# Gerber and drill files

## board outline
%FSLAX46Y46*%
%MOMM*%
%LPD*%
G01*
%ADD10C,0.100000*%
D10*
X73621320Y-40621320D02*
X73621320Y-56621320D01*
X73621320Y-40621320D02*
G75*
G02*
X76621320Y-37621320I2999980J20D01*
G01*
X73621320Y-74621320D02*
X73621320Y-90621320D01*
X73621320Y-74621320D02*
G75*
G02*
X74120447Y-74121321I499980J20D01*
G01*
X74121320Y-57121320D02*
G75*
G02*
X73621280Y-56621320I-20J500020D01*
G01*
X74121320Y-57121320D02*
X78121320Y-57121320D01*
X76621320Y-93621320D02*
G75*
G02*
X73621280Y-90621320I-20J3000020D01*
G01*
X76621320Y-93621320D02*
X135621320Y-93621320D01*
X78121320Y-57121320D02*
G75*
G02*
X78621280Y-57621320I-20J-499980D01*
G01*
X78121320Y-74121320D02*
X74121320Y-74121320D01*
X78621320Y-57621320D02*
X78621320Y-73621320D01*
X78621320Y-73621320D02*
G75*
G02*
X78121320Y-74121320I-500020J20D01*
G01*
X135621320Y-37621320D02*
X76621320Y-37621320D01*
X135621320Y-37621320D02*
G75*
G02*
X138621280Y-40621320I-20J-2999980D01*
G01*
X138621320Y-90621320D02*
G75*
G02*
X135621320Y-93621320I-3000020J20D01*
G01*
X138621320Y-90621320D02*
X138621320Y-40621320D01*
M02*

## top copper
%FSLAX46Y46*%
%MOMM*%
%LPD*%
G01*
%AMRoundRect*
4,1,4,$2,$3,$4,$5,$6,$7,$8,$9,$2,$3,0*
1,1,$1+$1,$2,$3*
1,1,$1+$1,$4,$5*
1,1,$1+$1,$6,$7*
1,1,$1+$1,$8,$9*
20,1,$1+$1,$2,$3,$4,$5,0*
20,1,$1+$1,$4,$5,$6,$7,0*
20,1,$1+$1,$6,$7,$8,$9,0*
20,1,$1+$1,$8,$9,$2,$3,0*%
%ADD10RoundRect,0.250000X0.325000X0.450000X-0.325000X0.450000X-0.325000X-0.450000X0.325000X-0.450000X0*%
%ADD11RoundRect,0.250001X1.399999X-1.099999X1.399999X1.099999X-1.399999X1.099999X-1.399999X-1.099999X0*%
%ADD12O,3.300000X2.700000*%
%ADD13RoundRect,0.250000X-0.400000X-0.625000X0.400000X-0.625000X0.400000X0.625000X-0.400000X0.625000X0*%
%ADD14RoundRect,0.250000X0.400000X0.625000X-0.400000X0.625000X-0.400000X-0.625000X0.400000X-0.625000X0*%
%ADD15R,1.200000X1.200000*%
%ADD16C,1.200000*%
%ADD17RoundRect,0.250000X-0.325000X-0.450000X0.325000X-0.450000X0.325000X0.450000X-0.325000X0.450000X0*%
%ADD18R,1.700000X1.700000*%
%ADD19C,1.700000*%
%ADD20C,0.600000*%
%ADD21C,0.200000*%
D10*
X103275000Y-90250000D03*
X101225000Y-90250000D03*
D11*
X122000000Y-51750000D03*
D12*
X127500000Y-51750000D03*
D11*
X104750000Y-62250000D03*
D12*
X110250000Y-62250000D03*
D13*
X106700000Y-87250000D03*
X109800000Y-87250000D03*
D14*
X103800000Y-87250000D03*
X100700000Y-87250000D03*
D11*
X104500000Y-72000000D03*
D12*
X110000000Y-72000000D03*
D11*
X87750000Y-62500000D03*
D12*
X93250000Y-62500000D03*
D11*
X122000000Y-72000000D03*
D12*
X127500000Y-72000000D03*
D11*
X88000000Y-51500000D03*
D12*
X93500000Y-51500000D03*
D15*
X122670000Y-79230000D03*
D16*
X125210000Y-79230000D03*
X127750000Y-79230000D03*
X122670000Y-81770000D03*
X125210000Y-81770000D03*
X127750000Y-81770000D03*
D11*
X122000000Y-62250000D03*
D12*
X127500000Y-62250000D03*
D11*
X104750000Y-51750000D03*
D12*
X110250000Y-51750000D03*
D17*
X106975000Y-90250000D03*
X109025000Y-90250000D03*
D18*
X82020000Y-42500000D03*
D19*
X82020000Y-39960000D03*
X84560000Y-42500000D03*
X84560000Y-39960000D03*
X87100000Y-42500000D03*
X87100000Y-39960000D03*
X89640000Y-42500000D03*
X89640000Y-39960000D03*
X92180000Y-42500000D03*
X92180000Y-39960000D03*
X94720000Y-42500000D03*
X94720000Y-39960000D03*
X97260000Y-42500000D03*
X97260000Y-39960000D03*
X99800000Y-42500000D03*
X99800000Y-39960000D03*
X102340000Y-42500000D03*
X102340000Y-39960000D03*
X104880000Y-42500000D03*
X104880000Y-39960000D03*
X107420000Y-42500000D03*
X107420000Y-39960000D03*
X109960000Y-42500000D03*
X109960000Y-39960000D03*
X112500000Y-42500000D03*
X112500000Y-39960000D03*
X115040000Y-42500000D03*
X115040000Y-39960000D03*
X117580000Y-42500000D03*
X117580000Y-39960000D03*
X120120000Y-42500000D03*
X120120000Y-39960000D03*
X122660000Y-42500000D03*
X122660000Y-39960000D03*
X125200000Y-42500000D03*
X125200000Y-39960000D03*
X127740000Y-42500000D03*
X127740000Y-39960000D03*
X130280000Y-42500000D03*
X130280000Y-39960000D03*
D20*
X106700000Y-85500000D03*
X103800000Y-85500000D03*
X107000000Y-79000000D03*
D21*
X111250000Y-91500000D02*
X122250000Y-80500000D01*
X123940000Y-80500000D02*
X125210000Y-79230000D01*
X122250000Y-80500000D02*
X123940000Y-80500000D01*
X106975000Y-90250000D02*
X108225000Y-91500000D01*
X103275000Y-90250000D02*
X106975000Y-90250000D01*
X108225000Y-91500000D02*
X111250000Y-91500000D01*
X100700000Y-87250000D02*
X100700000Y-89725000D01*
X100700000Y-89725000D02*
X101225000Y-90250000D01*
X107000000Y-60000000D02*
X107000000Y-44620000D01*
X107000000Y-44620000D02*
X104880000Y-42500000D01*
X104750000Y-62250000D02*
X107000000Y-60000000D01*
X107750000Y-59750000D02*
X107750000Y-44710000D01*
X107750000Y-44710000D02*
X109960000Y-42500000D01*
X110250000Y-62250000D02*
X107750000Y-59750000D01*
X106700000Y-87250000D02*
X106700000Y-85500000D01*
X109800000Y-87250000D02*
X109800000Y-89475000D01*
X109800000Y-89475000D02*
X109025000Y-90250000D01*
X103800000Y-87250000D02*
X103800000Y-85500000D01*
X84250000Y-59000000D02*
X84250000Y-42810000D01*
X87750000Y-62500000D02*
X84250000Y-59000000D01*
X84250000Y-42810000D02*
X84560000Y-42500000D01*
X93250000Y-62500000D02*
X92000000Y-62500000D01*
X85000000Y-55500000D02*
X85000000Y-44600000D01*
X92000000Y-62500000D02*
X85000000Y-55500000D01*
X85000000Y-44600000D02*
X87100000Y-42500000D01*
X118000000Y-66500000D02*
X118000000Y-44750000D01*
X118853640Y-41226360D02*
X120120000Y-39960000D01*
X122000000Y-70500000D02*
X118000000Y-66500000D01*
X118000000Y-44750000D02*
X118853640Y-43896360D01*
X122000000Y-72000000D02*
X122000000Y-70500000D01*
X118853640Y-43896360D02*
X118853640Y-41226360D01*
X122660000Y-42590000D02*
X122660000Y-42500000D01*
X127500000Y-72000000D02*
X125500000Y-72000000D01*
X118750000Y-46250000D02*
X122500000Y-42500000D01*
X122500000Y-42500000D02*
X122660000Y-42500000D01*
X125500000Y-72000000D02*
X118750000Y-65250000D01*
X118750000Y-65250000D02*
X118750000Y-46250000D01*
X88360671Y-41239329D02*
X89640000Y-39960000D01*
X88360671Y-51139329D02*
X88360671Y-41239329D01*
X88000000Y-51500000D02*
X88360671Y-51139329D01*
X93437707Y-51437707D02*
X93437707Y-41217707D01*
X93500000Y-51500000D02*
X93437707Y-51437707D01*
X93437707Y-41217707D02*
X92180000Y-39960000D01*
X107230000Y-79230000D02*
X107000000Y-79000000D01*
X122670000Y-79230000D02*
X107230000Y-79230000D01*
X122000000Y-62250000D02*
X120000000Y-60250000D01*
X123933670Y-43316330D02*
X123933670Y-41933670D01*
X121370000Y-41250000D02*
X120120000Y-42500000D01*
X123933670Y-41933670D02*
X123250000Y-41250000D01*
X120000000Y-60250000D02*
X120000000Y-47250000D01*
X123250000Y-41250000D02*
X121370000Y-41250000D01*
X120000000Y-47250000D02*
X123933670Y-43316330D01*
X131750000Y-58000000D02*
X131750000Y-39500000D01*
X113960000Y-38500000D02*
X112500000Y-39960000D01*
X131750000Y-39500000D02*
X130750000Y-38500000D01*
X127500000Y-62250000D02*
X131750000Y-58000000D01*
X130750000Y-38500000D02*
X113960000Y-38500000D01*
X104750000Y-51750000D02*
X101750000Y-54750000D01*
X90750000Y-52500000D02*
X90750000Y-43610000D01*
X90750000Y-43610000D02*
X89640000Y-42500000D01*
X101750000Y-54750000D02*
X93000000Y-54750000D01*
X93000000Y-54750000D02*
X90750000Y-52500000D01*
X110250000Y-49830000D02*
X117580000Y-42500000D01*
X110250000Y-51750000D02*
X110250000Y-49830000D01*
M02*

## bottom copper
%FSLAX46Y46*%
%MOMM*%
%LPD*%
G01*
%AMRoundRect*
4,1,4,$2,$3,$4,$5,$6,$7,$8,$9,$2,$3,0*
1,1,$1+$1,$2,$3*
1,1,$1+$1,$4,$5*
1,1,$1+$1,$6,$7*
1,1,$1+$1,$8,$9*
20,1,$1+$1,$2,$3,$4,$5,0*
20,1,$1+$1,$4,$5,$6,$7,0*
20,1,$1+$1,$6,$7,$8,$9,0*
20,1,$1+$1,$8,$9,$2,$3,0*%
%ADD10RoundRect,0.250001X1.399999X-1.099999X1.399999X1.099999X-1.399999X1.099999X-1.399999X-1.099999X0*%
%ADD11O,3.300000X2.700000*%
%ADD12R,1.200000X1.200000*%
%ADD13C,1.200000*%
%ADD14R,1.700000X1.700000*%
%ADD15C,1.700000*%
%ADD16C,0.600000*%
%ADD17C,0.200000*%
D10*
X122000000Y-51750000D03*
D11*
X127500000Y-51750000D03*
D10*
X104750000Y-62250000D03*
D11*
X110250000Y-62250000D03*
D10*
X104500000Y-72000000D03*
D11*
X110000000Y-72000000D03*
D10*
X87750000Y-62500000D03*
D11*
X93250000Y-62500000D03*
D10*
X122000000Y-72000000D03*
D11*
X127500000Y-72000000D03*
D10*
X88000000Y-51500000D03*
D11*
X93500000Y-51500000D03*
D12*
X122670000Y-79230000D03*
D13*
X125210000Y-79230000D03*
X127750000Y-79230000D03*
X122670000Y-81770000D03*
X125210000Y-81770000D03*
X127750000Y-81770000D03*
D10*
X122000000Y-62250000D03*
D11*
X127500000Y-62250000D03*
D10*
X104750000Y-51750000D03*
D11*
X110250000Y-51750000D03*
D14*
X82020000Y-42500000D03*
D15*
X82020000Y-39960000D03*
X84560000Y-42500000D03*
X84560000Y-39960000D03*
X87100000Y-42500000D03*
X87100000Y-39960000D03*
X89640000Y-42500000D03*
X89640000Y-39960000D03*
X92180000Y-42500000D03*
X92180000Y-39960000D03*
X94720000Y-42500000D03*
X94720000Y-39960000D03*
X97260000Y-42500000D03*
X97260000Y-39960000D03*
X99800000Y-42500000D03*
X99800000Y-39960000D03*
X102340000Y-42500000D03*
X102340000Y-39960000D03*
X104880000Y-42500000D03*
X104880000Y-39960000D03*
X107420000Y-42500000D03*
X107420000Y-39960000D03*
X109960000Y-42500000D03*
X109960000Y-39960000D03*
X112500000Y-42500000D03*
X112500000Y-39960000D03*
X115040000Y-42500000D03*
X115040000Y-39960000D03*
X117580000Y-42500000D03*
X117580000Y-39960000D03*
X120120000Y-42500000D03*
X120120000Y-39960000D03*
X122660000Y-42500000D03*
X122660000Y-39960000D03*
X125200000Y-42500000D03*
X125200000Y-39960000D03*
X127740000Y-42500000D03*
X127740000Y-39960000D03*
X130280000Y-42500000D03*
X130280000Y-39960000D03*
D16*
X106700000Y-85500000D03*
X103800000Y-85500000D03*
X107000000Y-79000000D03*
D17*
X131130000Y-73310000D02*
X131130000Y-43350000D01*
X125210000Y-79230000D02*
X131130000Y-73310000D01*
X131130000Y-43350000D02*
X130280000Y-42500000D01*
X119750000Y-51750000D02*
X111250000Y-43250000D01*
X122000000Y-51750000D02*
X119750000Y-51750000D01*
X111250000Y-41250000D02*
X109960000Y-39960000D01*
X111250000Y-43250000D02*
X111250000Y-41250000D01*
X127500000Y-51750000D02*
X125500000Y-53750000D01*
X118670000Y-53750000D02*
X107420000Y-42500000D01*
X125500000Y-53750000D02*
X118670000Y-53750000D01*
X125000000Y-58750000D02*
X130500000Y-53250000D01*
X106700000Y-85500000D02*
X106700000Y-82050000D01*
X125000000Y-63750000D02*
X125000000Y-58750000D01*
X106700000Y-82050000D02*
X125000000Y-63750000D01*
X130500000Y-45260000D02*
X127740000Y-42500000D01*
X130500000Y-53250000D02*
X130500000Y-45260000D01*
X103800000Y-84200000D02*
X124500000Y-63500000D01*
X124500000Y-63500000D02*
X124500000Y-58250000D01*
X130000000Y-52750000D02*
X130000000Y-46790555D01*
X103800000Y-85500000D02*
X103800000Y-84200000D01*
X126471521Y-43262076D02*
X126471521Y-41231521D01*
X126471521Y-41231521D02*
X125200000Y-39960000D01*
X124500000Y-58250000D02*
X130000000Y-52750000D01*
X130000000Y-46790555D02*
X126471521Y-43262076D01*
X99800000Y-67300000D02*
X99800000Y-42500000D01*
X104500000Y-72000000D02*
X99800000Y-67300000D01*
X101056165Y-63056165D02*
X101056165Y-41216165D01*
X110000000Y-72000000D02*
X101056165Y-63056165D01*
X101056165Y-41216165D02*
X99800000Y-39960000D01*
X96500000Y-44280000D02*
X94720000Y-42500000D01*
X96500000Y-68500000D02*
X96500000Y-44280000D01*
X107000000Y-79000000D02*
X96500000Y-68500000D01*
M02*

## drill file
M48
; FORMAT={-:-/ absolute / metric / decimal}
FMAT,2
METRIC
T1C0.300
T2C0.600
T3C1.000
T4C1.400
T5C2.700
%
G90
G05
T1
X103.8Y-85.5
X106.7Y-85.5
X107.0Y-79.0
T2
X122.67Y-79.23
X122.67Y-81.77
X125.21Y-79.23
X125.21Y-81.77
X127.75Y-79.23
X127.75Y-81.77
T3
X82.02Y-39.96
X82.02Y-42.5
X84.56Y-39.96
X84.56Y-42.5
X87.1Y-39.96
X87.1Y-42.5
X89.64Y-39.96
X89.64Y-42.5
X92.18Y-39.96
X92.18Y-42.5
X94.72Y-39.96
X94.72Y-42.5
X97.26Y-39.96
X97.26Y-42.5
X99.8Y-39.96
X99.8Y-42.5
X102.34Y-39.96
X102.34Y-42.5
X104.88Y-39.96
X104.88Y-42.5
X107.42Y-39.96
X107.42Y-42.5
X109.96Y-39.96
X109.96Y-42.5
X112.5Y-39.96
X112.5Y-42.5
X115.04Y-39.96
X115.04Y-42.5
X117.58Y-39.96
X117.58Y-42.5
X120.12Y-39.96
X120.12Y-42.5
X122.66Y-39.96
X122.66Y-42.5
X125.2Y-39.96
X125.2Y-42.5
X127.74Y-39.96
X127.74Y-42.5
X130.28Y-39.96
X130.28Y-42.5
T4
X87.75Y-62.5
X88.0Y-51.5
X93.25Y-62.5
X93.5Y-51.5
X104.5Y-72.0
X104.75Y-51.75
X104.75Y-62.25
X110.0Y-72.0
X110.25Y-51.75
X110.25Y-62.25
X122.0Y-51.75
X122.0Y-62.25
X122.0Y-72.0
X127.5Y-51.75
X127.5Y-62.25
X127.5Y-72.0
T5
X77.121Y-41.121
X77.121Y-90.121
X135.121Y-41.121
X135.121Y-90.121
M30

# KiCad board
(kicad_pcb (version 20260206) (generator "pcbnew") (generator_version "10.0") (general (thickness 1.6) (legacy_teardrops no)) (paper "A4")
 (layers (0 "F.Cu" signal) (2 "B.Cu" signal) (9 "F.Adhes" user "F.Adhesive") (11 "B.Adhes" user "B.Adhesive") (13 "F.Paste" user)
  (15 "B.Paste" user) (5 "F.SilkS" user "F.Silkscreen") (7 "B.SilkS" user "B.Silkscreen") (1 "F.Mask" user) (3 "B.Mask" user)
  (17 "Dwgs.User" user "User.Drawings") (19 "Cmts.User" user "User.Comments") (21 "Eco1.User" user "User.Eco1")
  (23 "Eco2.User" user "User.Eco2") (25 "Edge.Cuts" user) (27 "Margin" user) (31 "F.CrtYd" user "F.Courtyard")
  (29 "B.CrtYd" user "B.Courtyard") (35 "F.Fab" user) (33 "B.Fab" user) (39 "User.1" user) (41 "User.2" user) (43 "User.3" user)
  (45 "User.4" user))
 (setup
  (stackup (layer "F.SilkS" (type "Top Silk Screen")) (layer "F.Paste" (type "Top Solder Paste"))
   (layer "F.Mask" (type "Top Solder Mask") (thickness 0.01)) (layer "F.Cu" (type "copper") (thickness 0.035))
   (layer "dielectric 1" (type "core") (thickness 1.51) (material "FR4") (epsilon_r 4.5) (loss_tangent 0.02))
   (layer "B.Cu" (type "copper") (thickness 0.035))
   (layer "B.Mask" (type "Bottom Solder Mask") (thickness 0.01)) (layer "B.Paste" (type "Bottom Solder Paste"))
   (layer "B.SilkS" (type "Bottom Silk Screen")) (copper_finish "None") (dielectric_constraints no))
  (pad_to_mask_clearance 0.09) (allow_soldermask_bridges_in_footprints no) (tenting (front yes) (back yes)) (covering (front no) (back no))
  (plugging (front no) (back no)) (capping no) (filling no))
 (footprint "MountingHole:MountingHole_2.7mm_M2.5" (layer "F.Cu") (at 77.12132 41.12132)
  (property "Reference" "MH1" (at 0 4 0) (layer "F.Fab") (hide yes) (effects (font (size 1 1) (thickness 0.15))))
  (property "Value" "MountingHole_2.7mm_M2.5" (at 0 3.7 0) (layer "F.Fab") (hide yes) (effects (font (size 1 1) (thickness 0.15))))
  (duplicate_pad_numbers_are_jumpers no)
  (pad "" np_thru_hole circle (at 0 0) (size 2.7 2.7) (drill 2.7) (layers "*.Cu" "*.Mask")))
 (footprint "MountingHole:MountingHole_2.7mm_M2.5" (layer "F.Cu") (at 135.12132 41.12132)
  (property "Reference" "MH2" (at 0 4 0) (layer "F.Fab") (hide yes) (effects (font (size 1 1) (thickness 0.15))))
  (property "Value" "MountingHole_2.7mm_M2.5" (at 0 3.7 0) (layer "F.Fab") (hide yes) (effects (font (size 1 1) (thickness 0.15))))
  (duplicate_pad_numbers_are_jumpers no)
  (pad "" np_thru_hole circle (at 0 0) (size 2.7 2.7) (drill 2.7) (layers "*.Cu" "*.Mask")))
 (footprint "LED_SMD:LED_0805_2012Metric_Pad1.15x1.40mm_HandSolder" (layer "F.Cu") (at 102.25 90.25 180)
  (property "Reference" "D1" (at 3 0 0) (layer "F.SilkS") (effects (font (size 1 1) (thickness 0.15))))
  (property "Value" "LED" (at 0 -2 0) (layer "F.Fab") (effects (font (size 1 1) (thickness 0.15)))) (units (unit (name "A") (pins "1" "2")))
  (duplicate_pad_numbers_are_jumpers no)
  (pad "1" smd roundrect (at -1.025 0 180) (size 1.15 1.4) (layers "F.Cu" "F.Mask" "F.Paste") (roundrect_rratio 0.217391) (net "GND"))
  (pad "2" smd roundrect (at 1.025 0 180) (size 1.15 1.4) (layers "F.Cu" "F.Mask" "F.Paste") (roundrect_rratio 0.217391) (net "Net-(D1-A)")))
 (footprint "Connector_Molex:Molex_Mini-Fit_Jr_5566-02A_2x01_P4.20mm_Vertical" (layer "F.Cu") (at 122 51.75 90)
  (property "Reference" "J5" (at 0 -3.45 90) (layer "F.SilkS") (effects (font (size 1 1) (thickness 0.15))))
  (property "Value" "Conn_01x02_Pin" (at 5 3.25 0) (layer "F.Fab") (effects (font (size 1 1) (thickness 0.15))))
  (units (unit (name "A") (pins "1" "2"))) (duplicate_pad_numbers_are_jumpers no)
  (pad "1" thru_hole roundrect (at 0 0 90) (size 2.7 3.3) (drill 1.4) (layers "*.Cu" "*.Mask") (remove_unused_layers no)
   (roundrect_rratio 0.092593) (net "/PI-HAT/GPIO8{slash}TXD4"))
  (pad "2" thru_hole oval (at 0 5.5 90) (size 2.7 3.3) (drill 1.4) (layers "*.Cu" "*.Mask") (remove_unused_layers no)
   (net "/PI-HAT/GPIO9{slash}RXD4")))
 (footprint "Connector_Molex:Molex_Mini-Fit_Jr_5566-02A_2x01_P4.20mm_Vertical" (layer "F.Cu") (at 104.75 62.25 90)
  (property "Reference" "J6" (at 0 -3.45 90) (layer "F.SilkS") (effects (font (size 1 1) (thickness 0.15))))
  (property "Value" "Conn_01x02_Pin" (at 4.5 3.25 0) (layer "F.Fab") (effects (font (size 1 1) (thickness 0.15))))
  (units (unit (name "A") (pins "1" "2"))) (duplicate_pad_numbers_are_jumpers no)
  (pad "1" thru_hole roundrect (at 0 0 90) (size 2.7 3.3) (drill 1.4) (layers "*.Cu" "*.Mask") (remove_unused_layers no)
   (roundrect_rratio 0.092593) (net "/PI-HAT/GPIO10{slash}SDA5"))
  (pad "2" thru_hole oval (at 0 5.5 90) (size 2.7 3.3) (drill 1.4) (layers "*.Cu" "*.Mask") (remove_unused_layers no)
   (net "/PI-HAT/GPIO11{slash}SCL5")))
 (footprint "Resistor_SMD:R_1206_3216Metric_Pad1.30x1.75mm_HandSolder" (layer "F.Cu") (at 108.25 87.25)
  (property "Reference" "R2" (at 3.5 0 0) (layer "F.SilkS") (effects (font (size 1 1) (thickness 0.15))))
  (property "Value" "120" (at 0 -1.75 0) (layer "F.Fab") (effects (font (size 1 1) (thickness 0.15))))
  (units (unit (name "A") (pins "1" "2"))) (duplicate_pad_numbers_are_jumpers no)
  (pad "1" smd roundrect (at -1.55 0) (size 1.3 1.75) (layers "F.Cu" "F.Mask" "F.Paste") (roundrect_rratio 0.192308)
   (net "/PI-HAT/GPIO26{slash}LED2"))
  (pad "2" smd roundrect (at 1.55 0) (size 1.3 1.75) (layers "F.Cu" "F.Mask" "F.Paste") (roundrect_rratio 0.192308) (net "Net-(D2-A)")))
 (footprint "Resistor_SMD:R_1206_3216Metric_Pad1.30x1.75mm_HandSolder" (layer "F.Cu") (at 102.25 87.25 180)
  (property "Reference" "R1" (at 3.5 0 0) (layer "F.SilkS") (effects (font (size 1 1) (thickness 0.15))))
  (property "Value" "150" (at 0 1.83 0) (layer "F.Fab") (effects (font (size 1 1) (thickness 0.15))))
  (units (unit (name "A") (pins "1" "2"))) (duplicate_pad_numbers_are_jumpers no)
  (pad "1" smd roundrect (at -1.55 0 180) (size 1.3 1.75) (layers "F.Cu" "F.Mask" "F.Paste") (roundrect_rratio 0.192308)
   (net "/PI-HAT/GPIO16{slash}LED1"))
  (pad "2" smd roundrect (at 1.55 0 180) (size 1.3 1.75) (layers "F.Cu" "F.Mask" "F.Paste") (roundrect_rratio 0.192308) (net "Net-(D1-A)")))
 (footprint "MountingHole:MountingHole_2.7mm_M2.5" (layer "F.Cu") (at 77.12132 90.12132)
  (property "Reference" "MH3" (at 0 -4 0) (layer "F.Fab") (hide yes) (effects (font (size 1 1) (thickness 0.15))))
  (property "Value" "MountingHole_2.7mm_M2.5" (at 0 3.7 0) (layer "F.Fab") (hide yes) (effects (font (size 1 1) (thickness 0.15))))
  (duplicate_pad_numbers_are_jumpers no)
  (pad "" np_thru_hole circle (at 0 0) (size 2.7 2.7) (drill 2.7) (layers "*.Cu" "*.Mask")))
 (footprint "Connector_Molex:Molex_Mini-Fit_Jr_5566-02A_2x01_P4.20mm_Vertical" (layer "F.Cu") (at 104.5 72 90)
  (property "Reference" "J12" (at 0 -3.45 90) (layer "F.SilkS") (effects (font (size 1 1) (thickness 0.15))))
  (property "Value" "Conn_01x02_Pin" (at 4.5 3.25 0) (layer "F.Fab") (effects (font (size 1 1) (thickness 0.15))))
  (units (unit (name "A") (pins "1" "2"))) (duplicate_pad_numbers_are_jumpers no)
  (pad "1" thru_hole roundrect (at 0 0 90) (size 2.7 3.3) (drill 1.4) (layers "*.Cu" "*.Mask") (remove_unused_layers no)
   (roundrect_rratio 0.092593) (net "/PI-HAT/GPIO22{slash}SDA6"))
  (pad "2" thru_hole oval (at 0 5.5 90) (size 2.7 3.3) (drill 1.4) (layers "*.Cu" "*.Mask") (remove_unused_layers no)
   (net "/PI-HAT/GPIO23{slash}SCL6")))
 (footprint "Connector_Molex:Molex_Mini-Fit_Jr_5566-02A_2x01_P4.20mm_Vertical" (layer "F.Cu") (at 87.75 62.5 90)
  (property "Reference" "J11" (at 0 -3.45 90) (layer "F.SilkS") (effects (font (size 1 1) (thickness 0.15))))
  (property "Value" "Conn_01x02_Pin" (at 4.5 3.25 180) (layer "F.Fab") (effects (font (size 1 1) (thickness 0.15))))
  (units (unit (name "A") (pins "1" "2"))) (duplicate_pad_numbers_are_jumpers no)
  (pad "1" thru_hole roundrect (at 0 0 90) (size 2.7 3.3) (drill 1.4) (layers "*.Cu" "*.Mask") (remove_unused_layers no)
   (roundrect_rratio 0.092593) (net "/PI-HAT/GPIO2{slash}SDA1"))
  (pad "2" thru_hole oval (at 0 5.5 90) (size 2.7 3.3) (drill 1.4) (layers "*.Cu" "*.Mask") (remove_unused_layers no)
   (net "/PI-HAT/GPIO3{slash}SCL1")))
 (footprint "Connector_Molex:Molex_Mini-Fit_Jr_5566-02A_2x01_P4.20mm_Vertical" (layer "F.Cu") (at 122 72 90)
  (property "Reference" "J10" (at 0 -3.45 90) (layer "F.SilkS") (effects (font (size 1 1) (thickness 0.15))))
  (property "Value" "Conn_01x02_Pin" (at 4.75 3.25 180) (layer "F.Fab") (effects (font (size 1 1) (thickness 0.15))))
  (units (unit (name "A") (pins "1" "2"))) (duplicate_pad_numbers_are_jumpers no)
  (pad "1" thru_hole roundrect (at 0 0 90) (size 2.7 3.3) (drill 1.4) (layers "*.Cu" "*.Mask") (remove_unused_layers no)
   (roundrect_rratio 0.092593) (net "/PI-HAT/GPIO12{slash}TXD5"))
  (pad "2" thru_hole oval (at 0 5.5 90) (size 2.7 3.3) (drill 1.4) (layers "*.Cu" "*.Mask") (remove_unused_layers no)
   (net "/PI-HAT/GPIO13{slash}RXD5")))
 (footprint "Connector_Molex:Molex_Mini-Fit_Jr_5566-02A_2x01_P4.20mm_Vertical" (layer "F.Cu") (at 88 51.5 90)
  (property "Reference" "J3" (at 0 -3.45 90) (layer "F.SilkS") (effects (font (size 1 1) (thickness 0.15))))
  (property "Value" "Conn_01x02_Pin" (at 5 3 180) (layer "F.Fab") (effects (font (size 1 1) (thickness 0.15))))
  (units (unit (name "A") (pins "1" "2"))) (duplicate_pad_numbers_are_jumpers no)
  (pad "1" thru_hole roundrect (at 0 0 90) (size 2.7 3.3) (drill 1.4) (layers "*.Cu" "*.Mask") (remove_unused_layers no)
   (roundrect_rratio 0.092593) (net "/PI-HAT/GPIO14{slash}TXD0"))
  (pad "2" thru_hole oval (at 0 5.5 90) (size 2.7 3.3) (drill 1.4) (layers "*.Cu" "*.Mask") (remove_unused_layers no)
   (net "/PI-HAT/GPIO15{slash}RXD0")))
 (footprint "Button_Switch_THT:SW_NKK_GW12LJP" (layer "F.Cu") (at 122.67 79.23)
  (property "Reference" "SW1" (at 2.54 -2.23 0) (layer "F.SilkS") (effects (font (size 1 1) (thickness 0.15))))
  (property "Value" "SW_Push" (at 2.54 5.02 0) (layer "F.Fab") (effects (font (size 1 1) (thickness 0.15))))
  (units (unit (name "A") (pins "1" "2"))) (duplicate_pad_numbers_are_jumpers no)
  (pad "1" thru_hole rect (at 0 0) (size 1.2 1.2) (drill 0.6) (layers "*.Cu" "*.Mask") (remove_unused_layers no)
   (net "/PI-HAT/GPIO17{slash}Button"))
  (pad "2" thru_hole circle (at 2.54 0) (size 1.2 1.2) (drill 0.6) (layers "*.Cu" "*.Mask") (remove_unused_layers no) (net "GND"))
  (pad "3" thru_hole circle (at 5.08 0) (size 1.2 1.2) (drill 0.6) (layers "*.Cu" "*.Mask") (remove_unused_layers no))
  (pad "4" thru_hole circle (at 0 2.54) (size 1.2 1.2) (drill 0.6) (layers "*.Cu" "*.Mask") (remove_unused_layers no))
  (pad "5" thru_hole circle (at 2.54 2.54) (size 1.2 1.2) (drill 0.6) (layers "*.Cu" "*.Mask") (remove_unused_layers no))
  (pad "6" thru_hole circle (at 5.08 2.54) (size 1.2 1.2) (drill 0.6) (layers "*.Cu" "*.Mask") (remove_unused_layers no)))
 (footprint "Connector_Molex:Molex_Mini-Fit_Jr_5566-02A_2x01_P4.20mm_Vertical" (layer "F.Cu") (at 122 62.25 90)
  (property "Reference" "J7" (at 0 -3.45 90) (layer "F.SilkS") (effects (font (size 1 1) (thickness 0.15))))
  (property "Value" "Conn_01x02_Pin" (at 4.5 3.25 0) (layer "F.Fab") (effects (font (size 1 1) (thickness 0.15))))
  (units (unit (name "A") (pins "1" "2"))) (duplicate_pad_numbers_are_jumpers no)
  (pad "1" thru_hole roundrect (at 0 0 90) (size 2.7 3.3) (drill 1.4) (layers "*.Cu" "*.Mask") (remove_unused_layers no)
   (roundrect_rratio 0.092593) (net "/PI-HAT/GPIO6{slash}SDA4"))
  (pad "2" thru_hole oval (at 0 5.5 90) (size 2.7 3.3) (drill 1.4) (layers "*.Cu" "*.Mask") (remove_unused_layers no)
   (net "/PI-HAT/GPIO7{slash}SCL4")))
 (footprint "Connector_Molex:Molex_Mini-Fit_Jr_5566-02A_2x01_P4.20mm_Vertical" (layer "F.Cu") (at 104.75 51.75 90)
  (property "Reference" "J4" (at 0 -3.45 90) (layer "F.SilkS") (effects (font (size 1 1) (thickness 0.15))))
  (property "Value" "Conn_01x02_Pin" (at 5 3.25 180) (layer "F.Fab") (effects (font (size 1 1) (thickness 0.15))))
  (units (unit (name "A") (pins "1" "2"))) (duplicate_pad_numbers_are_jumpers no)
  (pad "1" thru_hole roundrect (at 0 0 90) (size 2.7 3.3) (drill 1.4) (layers "*.Cu" "*.Mask") (remove_unused_layers no)
   (roundrect_rratio 0.092593) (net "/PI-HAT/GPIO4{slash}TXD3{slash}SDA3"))
  (pad "2" thru_hole oval (at 0 5.5 90) (size 2.7 3.3) (drill 1.4) (layers "*.Cu" "*.Mask") (remove_unused_layers no)
   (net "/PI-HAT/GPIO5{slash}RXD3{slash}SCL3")))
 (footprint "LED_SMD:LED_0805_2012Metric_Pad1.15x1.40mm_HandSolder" (layer "F.Cu") (at 108 90.25)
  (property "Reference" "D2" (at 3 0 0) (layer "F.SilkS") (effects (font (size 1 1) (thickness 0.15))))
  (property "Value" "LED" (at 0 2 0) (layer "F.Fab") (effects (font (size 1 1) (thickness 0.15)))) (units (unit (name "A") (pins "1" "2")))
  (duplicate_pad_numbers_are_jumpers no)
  (pad "1" smd roundrect (at -1.025 0) (size 1.15 1.4) (layers "F.Cu" "F.Mask" "F.Paste") (roundrect_rratio 0.217391) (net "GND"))
  (pad "2" smd roundrect (at 1.025 0) (size 1.15 1.4) (layers "F.Cu" "F.Mask" "F.Paste") (roundrect_rratio 0.217391) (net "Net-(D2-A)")))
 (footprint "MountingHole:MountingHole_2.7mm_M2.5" (layer "F.Cu") (at 135.12132 90.12132)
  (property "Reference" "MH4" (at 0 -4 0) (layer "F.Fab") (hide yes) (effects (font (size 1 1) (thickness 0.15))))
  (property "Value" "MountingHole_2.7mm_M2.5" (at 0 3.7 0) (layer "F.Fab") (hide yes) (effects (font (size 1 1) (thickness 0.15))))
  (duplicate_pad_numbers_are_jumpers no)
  (pad "" np_thru_hole circle (at 0 0) (size 2.7 2.7) (drill 2.7) (layers "*.Cu" "*.Mask")))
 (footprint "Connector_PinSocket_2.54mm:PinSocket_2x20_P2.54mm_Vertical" (layer "B.Cu") (at 82.02 42.5 -90)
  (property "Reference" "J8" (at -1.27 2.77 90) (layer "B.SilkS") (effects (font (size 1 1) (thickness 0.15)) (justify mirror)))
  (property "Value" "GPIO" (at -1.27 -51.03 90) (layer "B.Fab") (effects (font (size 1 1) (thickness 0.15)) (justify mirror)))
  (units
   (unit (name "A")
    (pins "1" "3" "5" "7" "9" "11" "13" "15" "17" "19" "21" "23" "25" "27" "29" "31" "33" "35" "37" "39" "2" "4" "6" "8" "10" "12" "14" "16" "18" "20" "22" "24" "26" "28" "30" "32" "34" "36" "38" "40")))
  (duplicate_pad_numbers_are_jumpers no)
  (pad "1" thru_hole rect (at 0 0 270) (size 1.7 1.7) (drill 1) (layers "*.Cu" "*.Mask") (remove_unused_layers no)
   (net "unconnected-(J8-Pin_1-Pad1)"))
  (pad "2" thru_hole circle (at -2.54 0 270) (size 1.7 1.7) (drill 1) (layers "*.Cu" "*.Mask") (remove_unused_layers no)
   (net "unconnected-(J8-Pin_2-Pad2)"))
  (pad "3" thru_hole circle (at 0 -2.54 270) (size 1.7 1.7) (drill 1) (layers "*.Cu" "*.Mask") (remove_unused_layers no)
   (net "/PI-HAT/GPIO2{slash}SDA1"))
  (pad "4" thru_hole circle (at -2.54 -2.54 270) (size 1.7 1.7) (drill 1) (layers "*.Cu" "*.Mask") (remove_unused_layers no)
   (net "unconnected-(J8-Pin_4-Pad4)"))
  (pad "5" thru_hole circle (at 0 -5.08 270) (size 1.7 1.7) (drill 1) (layers "*.Cu" "*.Mask") (remove_unused_layers no)
   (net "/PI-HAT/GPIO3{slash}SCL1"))
  (pad "6" thru_hole circle (at -2.54 -5.08 270) (size 1.7 1.7) (drill 1) (layers "*.Cu" "*.Mask") (remove_unused_layers no) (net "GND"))
  (pad "7" thru_hole circle (at 0 -7.62 270) (size 1.7 1.7) (drill 1) (layers "*.Cu" "*.Mask") (remove_unused_layers no)
   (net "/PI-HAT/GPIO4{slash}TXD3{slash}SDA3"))
  (pad "8" thru_hole circle (at -2.54 -7.62 270) (size 1.7 1.7) (drill 1) (layers "*.Cu" "*.Mask") (remove_unused_layers no)
   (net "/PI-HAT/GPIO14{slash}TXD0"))
  (pad "9" thru_hole circle (at 0 -10.16 270) (size 1.7 1.7) (drill 1) (layers "*.Cu" "*.Mask") (remove_unused_layers no) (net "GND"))
  (pad "10" thru_hole circle (at -2.54 -10.16 270) (size 1.7 1.7) (drill 1) (layers "*.Cu" "*.Mask") (remove_unused_layers no)
   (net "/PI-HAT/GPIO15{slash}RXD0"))
  (pad "11" thru_hole circle (at 0 -12.7 270) (size 1.7 1.7) (drill 1) (layers "*.Cu" "*.Mask") (remove_unused_layers no)
   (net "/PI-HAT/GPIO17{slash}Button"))
  (pad "12" thru_hole circle (at -2.54 -12.7 270) (size 1.7 1.7) (drill 1) (layers "*.Cu" "*.Mask") (remove_unused_layers no)
   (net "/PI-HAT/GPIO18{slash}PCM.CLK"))
  (pad "13" thru_hole circle (at 0 -15.24 270) (size 1.7 1.7) (drill 1) (layers "*.Cu" "*.Mask") (remove_unused_layers no)
   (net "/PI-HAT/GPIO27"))
  (pad "14" thru_hole circle (at -2.54 -15.24 270) (size 1.7 1.7) (drill 1) (layers "*.Cu" "*.Mask") (remove_unused_layers no) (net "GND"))
  (pad "15" thru_hole circle (at 0 -17.78 270) (size 1.7 1.7) (drill 1) (layers "*.Cu" "*.Mask") (remove_unused_layers no)
   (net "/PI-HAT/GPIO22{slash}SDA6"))
  (pad "16" thru_hole circle (at -2.54 -17.78 270) (size 1.7 1.7) (drill 1) (layers "*.Cu" "*.Mask") (remove_unused_layers no)
   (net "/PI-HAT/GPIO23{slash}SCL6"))
  (pad "17" thru_hole circle (at 0 -20.32 270) (size 1.7 1.7) (drill 1) (layers "*.Cu" "*.Mask") (remove_unused_layers no)
   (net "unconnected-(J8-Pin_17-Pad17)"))
  (pad "18" thru_hole circle (at -2.54 -20.32 270) (size 1.7 1.7) (drill 1) (layers "*.Cu" "*.Mask") (remove_unused_layers no)
   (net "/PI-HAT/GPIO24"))
  (pad "19" thru_hole circle (at 0 -22.86 270) (size 1.7 1.7) (drill 1) (layers "*.Cu" "*.Mask") (remove_unused_layers no)
   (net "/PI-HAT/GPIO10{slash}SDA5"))
  (pad "20" thru_hole circle (at -2.54 -22.86 270) (size 1.7 1.7) (drill 1) (layers "*.Cu" "*.Mask") (remove_unused_layers no) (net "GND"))
  (pad "21" thru_hole circle (at 0 -25.4 270) (size 1.7 1.7) (drill 1) (layers "*.Cu" "*.Mask") (remove_unused_layers no)
   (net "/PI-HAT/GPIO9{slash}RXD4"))
  (pad "22" thru_hole circle (at -2.54 -25.4 270) (size 1.7 1.7) (drill 1) (layers "*.Cu" "*.Mask") (remove_unused_layers no)
   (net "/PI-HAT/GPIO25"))
  (pad "23" thru_hole circle (at 0 -27.94 270) (size 1.7 1.7) (drill 1) (layers "*.Cu" "*.Mask") (remove_unused_layers no)
   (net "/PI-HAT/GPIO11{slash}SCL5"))
  (pad "24" thru_hole circle (at -2.54 -27.94 270) (size 1.7 1.7) (drill 1) (layers "*.Cu" "*.Mask") (remove_unused_layers no)
   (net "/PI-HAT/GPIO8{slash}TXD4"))
  (pad "25" thru_hole circle (at 0 -30.48 270) (size 1.7 1.7) (drill 1) (layers "*.Cu" "*.Mask") (remove_unused_layers no) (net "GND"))
  (pad "26" thru_hole circle (at -2.54 -30.48 270) (size 1.7 1.7) (drill 1) (layers "*.Cu" "*.Mask") (remove_unused_layers no)
   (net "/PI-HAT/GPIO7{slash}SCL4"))
  (pad "27" thru_hole circle (at 0 -33.02 270) (size 1.7 1.7) (drill 1) (layers "*.Cu" "*.Mask") (remove_unused_layers no)
   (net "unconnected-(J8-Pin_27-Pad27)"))
  (pad "28" thru_hole circle (at -2.54 -33.02 270) (size 1.7 1.7) (drill 1) (layers "*.Cu" "*.Mask") (remove_unused_layers no)
   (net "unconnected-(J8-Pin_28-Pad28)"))
  (pad "29" thru_hole circle (at 0 -35.56 270) (size 1.7 1.7) (drill 1) (layers "*.Cu" "*.Mask") (remove_unused_layers no)
   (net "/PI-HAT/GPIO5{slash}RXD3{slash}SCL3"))
  (pad "30" thru_hole circle (at -2.54 -35.56 270) (size 1.7 1.7) (drill 1) (layers "*.Cu" "*.Mask") (remove_unused_layers no) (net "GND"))
  (pad "31" thru_hole circle (at 0 -38.1 270) (size 1.7 1.7) (drill 1) (layers "*.Cu" "*.Mask") (remove_unused_layers no)
   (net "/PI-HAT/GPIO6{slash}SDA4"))
  (pad "32" thru_hole circle (at -2.54 -38.1 270) (size 1.7 1.7) (drill 1) (layers "*.Cu" "*.Mask") (remove_unused_layers no)
   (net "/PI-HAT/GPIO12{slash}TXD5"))
  (pad "33" thru_hole circle (at 0 -40.64 270) (size 1.7 1.7) (drill 1) (layers "*.Cu" "*.Mask") (remove_unused_layers no)
   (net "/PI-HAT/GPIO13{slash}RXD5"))
  (pad "34" thru_hole circle (at -2.54 -40.64 270) (size 1.7 1.7) (drill 1) (layers "*.Cu" "*.Mask") (remove_unused_layers no) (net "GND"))
  (pad "35" thru_hole circle (at 0 -43.18 270) (size 1.7 1.7) (drill 1) (layers "*.Cu" "*.Mask") (remove_unused_layers no)
   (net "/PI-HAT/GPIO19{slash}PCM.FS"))
  (pad "36" thru_hole circle (at -2.54 -43.18 270) (size 1.7 1.7) (drill 1) (layers "*.Cu" "*.Mask") (remove_unused_layers no)
   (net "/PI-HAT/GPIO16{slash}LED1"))
  (pad "37" thru_hole circle (at 0 -45.72 270) (size 1.7 1.7) (drill 1) (layers "*.Cu" "*.Mask") (remove_unused_layers no)
   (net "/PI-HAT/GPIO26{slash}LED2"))
  (pad "38" thru_hole circle (at -2.54 -45.72 270) (size 1.7 1.7) (drill 1) (layers "*.Cu" "*.Mask") (remove_unused_layers no)
   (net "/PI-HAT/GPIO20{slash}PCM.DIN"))
  (pad "39" thru_hole circle (at 0 -48.26 270) (size 1.7 1.7) (drill 1) (layers "*.Cu" "*.Mask") (remove_unused_layers no) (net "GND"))
  (pad "40" thru_hole circle (at -2.54 -48.26 270) (size 1.7 1.7) (drill 1) (layers "*.Cu" "*.Mask") (remove_unused_layers no)
   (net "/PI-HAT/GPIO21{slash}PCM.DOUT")))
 (gr_line (start 73.62132 40.62132) (end 73.62132 56.62132) (stroke (width 0.1) (type solid)) (layer "Edge.Cuts"))
 (gr_arc (start 73.62132 40.62132) (mid 74.5 38.5) (end 76.62132 37.62132) (stroke (width 0.1) (type solid)) (layer "Edge.Cuts"))
 (gr_line (start 73.62132 74.62132) (end 73.62132 90.62132) (stroke (width 0.1) (type solid)) (layer "Edge.Cuts"))
 (gr_arc (start 73.62132 74.62132) (mid 73.767458 74.268075) (end 74.120447 74.121321) (stroke (width 0.1) (type solid)) (layer "Edge.Cuts"))
 (gr_arc (start 74.12132 57.12132) (mid 73.767767 56.974873) (end 73.62132 56.62132) (stroke (width 0.1) (type solid)) (layer "Edge.Cuts"))
 (gr_line (start 74.12132 57.12132) (end 78.12132 57.12132) (stroke (width 0.1) (type solid)) (layer "Edge.Cuts"))
 (gr_arc (start 76.62132 93.62132) (mid 74.5 92.74264) (end 73.62132 90.62132) (stroke (width 0.1) (type solid)) (layer "Edge.Cuts"))
 (gr_line (start 76.62132 93.62132) (end 135.62132 93.62132) (stroke (width 0.1) (type solid)) (layer "Edge.Cuts"))
 (gr_arc (start 78.12132 57.12132) (mid 78.474873 57.267767) (end 78.62132 57.62132) (stroke (width 0.1) (type solid)) (layer "Edge.Cuts"))
 (gr_line (start 78.12132 74.12132) (end 74.12132 74.12132) (stroke (width 0.1) (type solid)) (layer "Edge.Cuts"))
 (gr_line (start 78.62132 57.62132) (end 78.62132 73.62132) (stroke (width 0.1) (type solid)) (layer "Edge.Cuts"))
 (gr_arc (start 78.62132 73.62132) (mid 78.474873 73.974873) (end 78.12132 74.12132) (stroke (width 0.1) (type solid)) (layer "Edge.Cuts"))
 (gr_line (start 135.62132 37.62132) (end 76.62132 37.62132) (stroke (width 0.1) (type solid)) (layer "Edge.Cuts"))
 (gr_arc (start 135.62132 37.62132) (mid 137.74264 38.5) (end 138.62132 40.62132) (stroke (width 0.1) (type solid)) (layer "Edge.Cuts"))
 (gr_arc (start 138.62132 90.62132) (mid 137.74264 92.74264) (end 135.62132 93.62132) (stroke (width 0.1) (type solid)) (layer "Edge.Cuts"))
 (gr_line (start 138.62132 90.62132) (end 138.62132 40.62132) (stroke (width 0.1) (type solid)) (layer "Edge.Cuts"))
 (segment (start 111.25 91.5) (end 122.25 80.5) (width 0.2) (layer "F.Cu") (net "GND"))
 (segment (start 123.94 80.5) (end 125.21 79.23) (width 0.2) (layer "F.Cu") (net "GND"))
 (segment (start 122.25 80.5) (end 123.94 80.5) (width 0.2) (layer "F.Cu") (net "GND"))
 (segment (start 106.975 90.25) (end 108.225 91.5) (width 0.2) (layer "F.Cu") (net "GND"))
 (segment (start 103.275 90.25) (end 106.975 90.25) (width 0.2) (layer "F.Cu") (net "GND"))
 (segment (start 108.225 91.5) (end 111.25 91.5) (width 0.2) (layer "F.Cu") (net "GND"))
 (segment (start 131.13 73.31) (end 131.13 43.35) (width 0.2) (layer "B.Cu") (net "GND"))
 (segment (start 125.21 79.23) (end 131.13 73.31) (width 0.2) (layer "B.Cu") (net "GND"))
 (segment (start 131.13 43.35) (end 130.28 42.5) (width 0.2) (layer "B.Cu") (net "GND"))
 (segment (start 100.7 87.25) (end 100.7 89.725) (width 0.2) (layer "F.Cu") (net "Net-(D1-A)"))
 (segment (start 100.7 89.725) (end 101.225 90.25) (width 0.2) (layer "F.Cu") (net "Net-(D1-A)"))
 (segment (start 119.75 51.75) (end 111.25 43.25) (width 0.2) (layer "B.Cu") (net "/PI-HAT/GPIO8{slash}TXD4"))
 (segment (start 122 51.75) (end 119.75 51.75) (width 0.2) (layer "B.Cu") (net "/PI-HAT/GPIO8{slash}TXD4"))
 (segment (start 111.25 41.25) (end 109.96 39.96) (width 0.2) (layer "B.Cu") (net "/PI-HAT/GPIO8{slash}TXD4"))
 (segment (start 111.25 43.25) (end 111.25 41.25) (width 0.2) (layer "B.Cu") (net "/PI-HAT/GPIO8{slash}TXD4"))
 (segment (start 127.5 51.75) (end 125.5 53.75) (width 0.2) (layer "B.Cu") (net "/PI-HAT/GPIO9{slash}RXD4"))
 (segment (start 118.67 53.75) (end 107.42 42.5) (width 0.2) (layer "B.Cu") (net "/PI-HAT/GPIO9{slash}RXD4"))
 (segment (start 125.5 53.75) (end 118.67 53.75) (width 0.2) (layer "B.Cu") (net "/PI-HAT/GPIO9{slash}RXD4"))
 (segment (start 107 60) (end 107 44.62) (width 0.2) (layer "F.Cu") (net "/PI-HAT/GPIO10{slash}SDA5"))
 (segment (start 107 44.62) (end 104.88 42.5) (width 0.2) (layer "F.Cu") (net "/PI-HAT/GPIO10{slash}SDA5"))
 (segment (start 104.75 62.25) (end 107 60) (width 0.2) (layer "F.Cu") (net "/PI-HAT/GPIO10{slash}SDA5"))
 (segment (start 107.75 59.75) (end 107.75 44.71) (width 0.2) (layer "F.Cu") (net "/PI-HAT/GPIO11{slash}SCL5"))
 (segment (start 107.75 44.71) (end 109.96 42.5) (width 0.2) (layer "F.Cu") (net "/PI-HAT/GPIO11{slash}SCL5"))
 (segment (start 110.25 62.25) (end 107.75 59.75) (width 0.2) (layer "F.Cu") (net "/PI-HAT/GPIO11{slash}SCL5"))
 (segment (start 106.7 87.25) (end 106.7 85.5) (width 0.2) (layer "F.Cu") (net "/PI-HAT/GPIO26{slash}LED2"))
 (via (at 106.7 85.5) (size 0.6) (drill 0.3) (layers "F.Cu" "B.Cu") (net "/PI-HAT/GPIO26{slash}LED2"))
 (segment (start 125 58.75) (end 130.5 53.25) (width 0.2) (layer "B.Cu") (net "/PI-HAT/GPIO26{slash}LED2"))
 (segment (start 106.7 85.5) (end 106.7 82.05) (width 0.2) (layer "B.Cu") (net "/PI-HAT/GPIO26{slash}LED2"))
 (segment (start 125 63.75) (end 125 58.75) (width 0.2) (layer "B.Cu") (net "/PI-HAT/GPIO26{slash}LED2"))
 (segment (start 106.7 82.05) (end 125 63.75) (width 0.2) (layer "B.Cu") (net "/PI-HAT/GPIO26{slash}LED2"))
 (segment (start 130.5 45.26) (end 127.74 42.5) (width 0.2) (layer "B.Cu") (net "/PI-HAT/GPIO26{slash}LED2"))
 (segment (start 130.5 53.25) (end 130.5 45.26) (width 0.2) (layer "B.Cu") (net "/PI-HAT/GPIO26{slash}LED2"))
 (segment (start 109.8 87.25) (end 109.8 89.475) (width 0.2) (layer "F.Cu") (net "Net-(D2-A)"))
 (segment (start 109.8 89.475) (end 109.025 90.25) (width 0.2) (layer "F.Cu") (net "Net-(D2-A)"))
 (segment (start 103.8 87.25) (end 103.8 85.5) (width 0.2) (layer "F.Cu") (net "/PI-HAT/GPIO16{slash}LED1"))
 (via (at 103.8 85.5) (size 0.6) (drill 0.3) (layers "F.Cu" "B.Cu") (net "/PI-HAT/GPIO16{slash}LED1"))
 (segment (start 103.8 84.2) (end 124.5 63.5) (width 0.2) (layer "B.Cu") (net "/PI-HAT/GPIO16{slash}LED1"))
 (segment (start 124.5 63.5) (end 124.5 58.25) (width 0.2) (layer "B.Cu") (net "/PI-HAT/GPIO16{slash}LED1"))
 (segment (start 130 52.75) (end 130 46.790555) (width 0.2) (layer "B.Cu") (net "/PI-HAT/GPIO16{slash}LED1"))
 (segment (start 103.8 85.5) (end 103.8 84.2) (width 0.2) (layer "B.Cu") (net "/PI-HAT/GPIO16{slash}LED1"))
 (segment (start 126.471521 43.262076) (end 126.471521 41.231521) (width 0.2) (layer "B.Cu") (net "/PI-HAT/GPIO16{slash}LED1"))
 (segment (start 126.471521 41.231521) (end 125.2 39.96) (width 0.2) (layer "B.Cu") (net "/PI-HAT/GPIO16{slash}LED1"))
 (segment (start 124.5 58.25) (end 130 52.75) (width 0.2) (layer "B.Cu") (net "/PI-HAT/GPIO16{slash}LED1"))
 (segment (start 130 46.790555) (end 126.471521 43.262076) (width 0.2) (layer "B.Cu") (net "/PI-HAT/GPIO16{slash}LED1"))
 (segment (start 99.8 67.3) (end 99.8 42.5) (width 0.2) (layer "B.Cu") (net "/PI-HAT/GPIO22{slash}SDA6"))
 (segment (start 104.5 72) (end 99.8 67.3) (width 0.2) (layer "B.Cu") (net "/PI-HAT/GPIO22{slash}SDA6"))
 (segment (start 101.056165 63.056165) (end 101.056165 41.216165) (width 0.2) (layer "B.Cu") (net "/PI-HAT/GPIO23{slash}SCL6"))
 (segment (start 110 72) (end 101.056165 63.056165) (width 0.2) (layer "B.Cu") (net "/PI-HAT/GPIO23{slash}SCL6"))
 (segment (start 101.056165 41.216165) (end 99.8 39.96) (width 0.2) (layer "B.Cu") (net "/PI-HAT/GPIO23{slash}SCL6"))
 (segment (start 84.25 59) (end 84.25 42.81) (width 0.2) (layer "F.Cu") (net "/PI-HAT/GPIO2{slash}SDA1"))
 (segment (start 87.75 62.5) (end 84.25 59) (width 0.2) (layer "F.Cu") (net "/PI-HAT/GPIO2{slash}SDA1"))
 (segment (start 84.25 42.81) (end 84.56 42.5) (width 0.2) (layer "F.Cu") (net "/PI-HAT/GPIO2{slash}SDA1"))
 (segment (start 93.25 62.5) (end 92 62.5) (width 0.2) (layer "F.Cu") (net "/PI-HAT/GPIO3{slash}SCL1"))
 (segment (start 85 55.5) (end 85 44.6) (width 0.2) (layer "F.Cu") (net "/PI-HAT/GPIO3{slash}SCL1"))
 (segment (start 92 62.5) (end 85 55.5) (width 0.2) (layer "F.Cu") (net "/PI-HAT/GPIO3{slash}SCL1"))
 (segment (start 85 44.6) (end 87.1 42.5) (width 0.2) (layer "F.Cu") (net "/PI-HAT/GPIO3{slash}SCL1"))
 (segment (start 118 66.5) (end 118 44.75) (width 0.2) (layer "F.Cu") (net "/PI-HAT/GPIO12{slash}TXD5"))
 (segment (start 118.85364 41.22636) (end 120.12 39.96) (width 0.2) (layer "F.Cu") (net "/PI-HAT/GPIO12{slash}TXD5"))
 (segment (start 122 70.5) (end 118 66.5) (width 0.2) (layer "F.Cu") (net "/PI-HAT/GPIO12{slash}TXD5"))
 (segment (start 118 44.75) (end 118.85364 43.89636) (width 0.2) (layer "F.Cu") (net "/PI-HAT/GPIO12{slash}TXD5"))
 (segment (start 122 72) (end 122 70.5) (width 0.2) (layer "F.Cu") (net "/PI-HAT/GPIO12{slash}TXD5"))
 (segment (start 118.85364 43.89636) (end 118.85364 41.22636) (width 0.2) (layer "F.Cu") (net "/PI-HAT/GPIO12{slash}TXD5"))
 (segment (start 122.66 42.59) (end 122.66 42.5) (width 0.2) (layer "F.Cu") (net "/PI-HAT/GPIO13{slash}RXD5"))
 (segment (start 127.5 72) (end 125.5 72) (width 0.2) (layer "F.Cu") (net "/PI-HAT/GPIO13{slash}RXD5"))
 (segment (start 118.75 46.25) (end 122.5 42.5) (width 0.2) (layer "F.Cu") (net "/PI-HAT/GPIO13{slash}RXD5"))
 (segment (start 122.5 42.5) (end 122.66 42.5) (width 0.2) (layer "F.Cu") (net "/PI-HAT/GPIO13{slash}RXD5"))
 (segment (start 125.5 72) (end 118.75 65.25) (width 0.2) (layer "F.Cu") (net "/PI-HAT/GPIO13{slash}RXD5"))
 (segment (start 118.75 65.25) (end 118.75 46.25) (width 0.2) (layer "F.Cu") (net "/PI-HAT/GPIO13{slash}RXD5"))
 (segment (start 88.360671 41.239329) (end 89.64 39.96) (width 0.2) (layer "F.Cu") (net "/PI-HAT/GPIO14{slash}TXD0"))
 (segment (start 88.360671 51.139329) (end 88.360671 41.239329) (width 0.2) (layer "F.Cu") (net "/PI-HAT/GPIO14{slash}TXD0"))
 (segment (start 88 51.5) (end 88.360671 51.139329) (width 0.2) (layer "F.Cu") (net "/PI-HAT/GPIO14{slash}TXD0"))
 (segment (start 93.437707 51.437707) (end 93.437707 41.217707) (width 0.2) (layer "F.Cu") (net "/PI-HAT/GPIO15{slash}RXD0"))
 (segment (start 93.5 51.5) (end 93.437707 51.437707) (width 0.2) (layer "F.Cu") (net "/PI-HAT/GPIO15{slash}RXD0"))
 (segment (start 93.437707 41.217707) (end 92.18 39.96) (width 0.2) (layer "F.Cu") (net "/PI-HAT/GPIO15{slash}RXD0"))
 (segment (start 107.23 79.23) (end 107 79) (width 0.2) (layer "F.Cu") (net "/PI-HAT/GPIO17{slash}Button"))
 (segment (start 122.67 79.23) (end 107.23 79.23) (width 0.2) (layer "F.Cu") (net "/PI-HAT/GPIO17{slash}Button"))
 (via (at 107 79) (size 0.6) (drill 0.3) (layers "F.Cu" "B.Cu") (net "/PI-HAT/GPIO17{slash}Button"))
 (segment (start 96.5 44.28) (end 94.72 42.5) (width 0.2) (layer "B.Cu") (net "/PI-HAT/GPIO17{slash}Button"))
 (segment (start 96.5 68.5) (end 96.5 44.28) (width 0.2) (layer "B.Cu") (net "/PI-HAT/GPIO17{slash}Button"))
 (segment (start 107 79) (end 96.5 68.5) (width 0.2) (layer "B.Cu") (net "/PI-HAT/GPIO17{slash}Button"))
 (segment (start 122 62.25) (end 120 60.25) (width 0.2) (layer "F.Cu") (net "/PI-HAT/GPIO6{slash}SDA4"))
 (segment (start 123.93367 43.31633) (end 123.93367 41.93367) (width 0.2) (layer "F.Cu") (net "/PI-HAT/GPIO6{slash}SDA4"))
 (segment (start 121.37 41.25) (end 120.12 42.5) (width 0.2) (layer "F.Cu") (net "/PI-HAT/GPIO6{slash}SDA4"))
 (segment (start 123.93367 41.93367) (end 123.25 41.25) (width 0.2) (layer "F.Cu") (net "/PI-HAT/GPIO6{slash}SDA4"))
 (segment (start 120 60.25) (end 120 47.25) (width 0.2) (layer "F.Cu") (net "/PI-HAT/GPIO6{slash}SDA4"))
 (segment (start 123.25 41.25) (end 121.37 41.25) (width 0.2) (layer "F.Cu") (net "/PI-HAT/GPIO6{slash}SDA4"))
 (segment (start 120 47.25) (end 123.93367 43.31633) (width 0.2) (layer "F.Cu") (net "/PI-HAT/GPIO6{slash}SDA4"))
 (segment (start 131.75 58) (end 131.75 39.5) (width 0.2) (layer "F.Cu") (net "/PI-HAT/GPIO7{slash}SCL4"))
 (segment (start 113.96 38.5) (end 112.5 39.96) (width 0.2) (layer "F.Cu") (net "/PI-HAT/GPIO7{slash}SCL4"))
 (segment (start 131.75 39.5) (end 130.75 38.5) (width 0.2) (layer "F.Cu") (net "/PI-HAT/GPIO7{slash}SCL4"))
 (segment (start 127.5 62.25) (end 131.75 58) (width 0.2) (layer "F.Cu") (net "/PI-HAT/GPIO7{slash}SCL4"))
 (segment (start 130.75 38.5) (end 113.96 38.5) (width 0.2) (layer "F.Cu") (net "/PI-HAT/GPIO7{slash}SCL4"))
 (segment (start 104.75 51.75) (end 101.75 54.75) (width 0.2) (layer "F.Cu") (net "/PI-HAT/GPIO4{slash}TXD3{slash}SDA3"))
 (segment (start 90.75 52.5) (end 90.75 43.61) (width 0.2) (layer "F.Cu") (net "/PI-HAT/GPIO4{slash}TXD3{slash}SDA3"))
 (segment (start 90.75 43.61) (end 89.64 42.5) (width 0.2) (layer "F.Cu") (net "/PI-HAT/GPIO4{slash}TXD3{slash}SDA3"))
 (segment (start 101.75 54.75) (end 93 54.75) (width 0.2) (layer "F.Cu") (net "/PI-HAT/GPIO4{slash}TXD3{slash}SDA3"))
 (segment (start 93 54.75) (end 90.75 52.5) (width 0.2) (layer "F.Cu") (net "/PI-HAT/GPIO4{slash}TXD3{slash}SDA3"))
 (segment (start 110.25 49.83) (end 117.58 42.5) (width 0.2) (layer "F.Cu") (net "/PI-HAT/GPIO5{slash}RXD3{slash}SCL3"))
 (segment (start 110.25 51.75) (end 110.25 49.83) (width 0.2) (layer "F.Cu") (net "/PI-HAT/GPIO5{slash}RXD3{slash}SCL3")))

